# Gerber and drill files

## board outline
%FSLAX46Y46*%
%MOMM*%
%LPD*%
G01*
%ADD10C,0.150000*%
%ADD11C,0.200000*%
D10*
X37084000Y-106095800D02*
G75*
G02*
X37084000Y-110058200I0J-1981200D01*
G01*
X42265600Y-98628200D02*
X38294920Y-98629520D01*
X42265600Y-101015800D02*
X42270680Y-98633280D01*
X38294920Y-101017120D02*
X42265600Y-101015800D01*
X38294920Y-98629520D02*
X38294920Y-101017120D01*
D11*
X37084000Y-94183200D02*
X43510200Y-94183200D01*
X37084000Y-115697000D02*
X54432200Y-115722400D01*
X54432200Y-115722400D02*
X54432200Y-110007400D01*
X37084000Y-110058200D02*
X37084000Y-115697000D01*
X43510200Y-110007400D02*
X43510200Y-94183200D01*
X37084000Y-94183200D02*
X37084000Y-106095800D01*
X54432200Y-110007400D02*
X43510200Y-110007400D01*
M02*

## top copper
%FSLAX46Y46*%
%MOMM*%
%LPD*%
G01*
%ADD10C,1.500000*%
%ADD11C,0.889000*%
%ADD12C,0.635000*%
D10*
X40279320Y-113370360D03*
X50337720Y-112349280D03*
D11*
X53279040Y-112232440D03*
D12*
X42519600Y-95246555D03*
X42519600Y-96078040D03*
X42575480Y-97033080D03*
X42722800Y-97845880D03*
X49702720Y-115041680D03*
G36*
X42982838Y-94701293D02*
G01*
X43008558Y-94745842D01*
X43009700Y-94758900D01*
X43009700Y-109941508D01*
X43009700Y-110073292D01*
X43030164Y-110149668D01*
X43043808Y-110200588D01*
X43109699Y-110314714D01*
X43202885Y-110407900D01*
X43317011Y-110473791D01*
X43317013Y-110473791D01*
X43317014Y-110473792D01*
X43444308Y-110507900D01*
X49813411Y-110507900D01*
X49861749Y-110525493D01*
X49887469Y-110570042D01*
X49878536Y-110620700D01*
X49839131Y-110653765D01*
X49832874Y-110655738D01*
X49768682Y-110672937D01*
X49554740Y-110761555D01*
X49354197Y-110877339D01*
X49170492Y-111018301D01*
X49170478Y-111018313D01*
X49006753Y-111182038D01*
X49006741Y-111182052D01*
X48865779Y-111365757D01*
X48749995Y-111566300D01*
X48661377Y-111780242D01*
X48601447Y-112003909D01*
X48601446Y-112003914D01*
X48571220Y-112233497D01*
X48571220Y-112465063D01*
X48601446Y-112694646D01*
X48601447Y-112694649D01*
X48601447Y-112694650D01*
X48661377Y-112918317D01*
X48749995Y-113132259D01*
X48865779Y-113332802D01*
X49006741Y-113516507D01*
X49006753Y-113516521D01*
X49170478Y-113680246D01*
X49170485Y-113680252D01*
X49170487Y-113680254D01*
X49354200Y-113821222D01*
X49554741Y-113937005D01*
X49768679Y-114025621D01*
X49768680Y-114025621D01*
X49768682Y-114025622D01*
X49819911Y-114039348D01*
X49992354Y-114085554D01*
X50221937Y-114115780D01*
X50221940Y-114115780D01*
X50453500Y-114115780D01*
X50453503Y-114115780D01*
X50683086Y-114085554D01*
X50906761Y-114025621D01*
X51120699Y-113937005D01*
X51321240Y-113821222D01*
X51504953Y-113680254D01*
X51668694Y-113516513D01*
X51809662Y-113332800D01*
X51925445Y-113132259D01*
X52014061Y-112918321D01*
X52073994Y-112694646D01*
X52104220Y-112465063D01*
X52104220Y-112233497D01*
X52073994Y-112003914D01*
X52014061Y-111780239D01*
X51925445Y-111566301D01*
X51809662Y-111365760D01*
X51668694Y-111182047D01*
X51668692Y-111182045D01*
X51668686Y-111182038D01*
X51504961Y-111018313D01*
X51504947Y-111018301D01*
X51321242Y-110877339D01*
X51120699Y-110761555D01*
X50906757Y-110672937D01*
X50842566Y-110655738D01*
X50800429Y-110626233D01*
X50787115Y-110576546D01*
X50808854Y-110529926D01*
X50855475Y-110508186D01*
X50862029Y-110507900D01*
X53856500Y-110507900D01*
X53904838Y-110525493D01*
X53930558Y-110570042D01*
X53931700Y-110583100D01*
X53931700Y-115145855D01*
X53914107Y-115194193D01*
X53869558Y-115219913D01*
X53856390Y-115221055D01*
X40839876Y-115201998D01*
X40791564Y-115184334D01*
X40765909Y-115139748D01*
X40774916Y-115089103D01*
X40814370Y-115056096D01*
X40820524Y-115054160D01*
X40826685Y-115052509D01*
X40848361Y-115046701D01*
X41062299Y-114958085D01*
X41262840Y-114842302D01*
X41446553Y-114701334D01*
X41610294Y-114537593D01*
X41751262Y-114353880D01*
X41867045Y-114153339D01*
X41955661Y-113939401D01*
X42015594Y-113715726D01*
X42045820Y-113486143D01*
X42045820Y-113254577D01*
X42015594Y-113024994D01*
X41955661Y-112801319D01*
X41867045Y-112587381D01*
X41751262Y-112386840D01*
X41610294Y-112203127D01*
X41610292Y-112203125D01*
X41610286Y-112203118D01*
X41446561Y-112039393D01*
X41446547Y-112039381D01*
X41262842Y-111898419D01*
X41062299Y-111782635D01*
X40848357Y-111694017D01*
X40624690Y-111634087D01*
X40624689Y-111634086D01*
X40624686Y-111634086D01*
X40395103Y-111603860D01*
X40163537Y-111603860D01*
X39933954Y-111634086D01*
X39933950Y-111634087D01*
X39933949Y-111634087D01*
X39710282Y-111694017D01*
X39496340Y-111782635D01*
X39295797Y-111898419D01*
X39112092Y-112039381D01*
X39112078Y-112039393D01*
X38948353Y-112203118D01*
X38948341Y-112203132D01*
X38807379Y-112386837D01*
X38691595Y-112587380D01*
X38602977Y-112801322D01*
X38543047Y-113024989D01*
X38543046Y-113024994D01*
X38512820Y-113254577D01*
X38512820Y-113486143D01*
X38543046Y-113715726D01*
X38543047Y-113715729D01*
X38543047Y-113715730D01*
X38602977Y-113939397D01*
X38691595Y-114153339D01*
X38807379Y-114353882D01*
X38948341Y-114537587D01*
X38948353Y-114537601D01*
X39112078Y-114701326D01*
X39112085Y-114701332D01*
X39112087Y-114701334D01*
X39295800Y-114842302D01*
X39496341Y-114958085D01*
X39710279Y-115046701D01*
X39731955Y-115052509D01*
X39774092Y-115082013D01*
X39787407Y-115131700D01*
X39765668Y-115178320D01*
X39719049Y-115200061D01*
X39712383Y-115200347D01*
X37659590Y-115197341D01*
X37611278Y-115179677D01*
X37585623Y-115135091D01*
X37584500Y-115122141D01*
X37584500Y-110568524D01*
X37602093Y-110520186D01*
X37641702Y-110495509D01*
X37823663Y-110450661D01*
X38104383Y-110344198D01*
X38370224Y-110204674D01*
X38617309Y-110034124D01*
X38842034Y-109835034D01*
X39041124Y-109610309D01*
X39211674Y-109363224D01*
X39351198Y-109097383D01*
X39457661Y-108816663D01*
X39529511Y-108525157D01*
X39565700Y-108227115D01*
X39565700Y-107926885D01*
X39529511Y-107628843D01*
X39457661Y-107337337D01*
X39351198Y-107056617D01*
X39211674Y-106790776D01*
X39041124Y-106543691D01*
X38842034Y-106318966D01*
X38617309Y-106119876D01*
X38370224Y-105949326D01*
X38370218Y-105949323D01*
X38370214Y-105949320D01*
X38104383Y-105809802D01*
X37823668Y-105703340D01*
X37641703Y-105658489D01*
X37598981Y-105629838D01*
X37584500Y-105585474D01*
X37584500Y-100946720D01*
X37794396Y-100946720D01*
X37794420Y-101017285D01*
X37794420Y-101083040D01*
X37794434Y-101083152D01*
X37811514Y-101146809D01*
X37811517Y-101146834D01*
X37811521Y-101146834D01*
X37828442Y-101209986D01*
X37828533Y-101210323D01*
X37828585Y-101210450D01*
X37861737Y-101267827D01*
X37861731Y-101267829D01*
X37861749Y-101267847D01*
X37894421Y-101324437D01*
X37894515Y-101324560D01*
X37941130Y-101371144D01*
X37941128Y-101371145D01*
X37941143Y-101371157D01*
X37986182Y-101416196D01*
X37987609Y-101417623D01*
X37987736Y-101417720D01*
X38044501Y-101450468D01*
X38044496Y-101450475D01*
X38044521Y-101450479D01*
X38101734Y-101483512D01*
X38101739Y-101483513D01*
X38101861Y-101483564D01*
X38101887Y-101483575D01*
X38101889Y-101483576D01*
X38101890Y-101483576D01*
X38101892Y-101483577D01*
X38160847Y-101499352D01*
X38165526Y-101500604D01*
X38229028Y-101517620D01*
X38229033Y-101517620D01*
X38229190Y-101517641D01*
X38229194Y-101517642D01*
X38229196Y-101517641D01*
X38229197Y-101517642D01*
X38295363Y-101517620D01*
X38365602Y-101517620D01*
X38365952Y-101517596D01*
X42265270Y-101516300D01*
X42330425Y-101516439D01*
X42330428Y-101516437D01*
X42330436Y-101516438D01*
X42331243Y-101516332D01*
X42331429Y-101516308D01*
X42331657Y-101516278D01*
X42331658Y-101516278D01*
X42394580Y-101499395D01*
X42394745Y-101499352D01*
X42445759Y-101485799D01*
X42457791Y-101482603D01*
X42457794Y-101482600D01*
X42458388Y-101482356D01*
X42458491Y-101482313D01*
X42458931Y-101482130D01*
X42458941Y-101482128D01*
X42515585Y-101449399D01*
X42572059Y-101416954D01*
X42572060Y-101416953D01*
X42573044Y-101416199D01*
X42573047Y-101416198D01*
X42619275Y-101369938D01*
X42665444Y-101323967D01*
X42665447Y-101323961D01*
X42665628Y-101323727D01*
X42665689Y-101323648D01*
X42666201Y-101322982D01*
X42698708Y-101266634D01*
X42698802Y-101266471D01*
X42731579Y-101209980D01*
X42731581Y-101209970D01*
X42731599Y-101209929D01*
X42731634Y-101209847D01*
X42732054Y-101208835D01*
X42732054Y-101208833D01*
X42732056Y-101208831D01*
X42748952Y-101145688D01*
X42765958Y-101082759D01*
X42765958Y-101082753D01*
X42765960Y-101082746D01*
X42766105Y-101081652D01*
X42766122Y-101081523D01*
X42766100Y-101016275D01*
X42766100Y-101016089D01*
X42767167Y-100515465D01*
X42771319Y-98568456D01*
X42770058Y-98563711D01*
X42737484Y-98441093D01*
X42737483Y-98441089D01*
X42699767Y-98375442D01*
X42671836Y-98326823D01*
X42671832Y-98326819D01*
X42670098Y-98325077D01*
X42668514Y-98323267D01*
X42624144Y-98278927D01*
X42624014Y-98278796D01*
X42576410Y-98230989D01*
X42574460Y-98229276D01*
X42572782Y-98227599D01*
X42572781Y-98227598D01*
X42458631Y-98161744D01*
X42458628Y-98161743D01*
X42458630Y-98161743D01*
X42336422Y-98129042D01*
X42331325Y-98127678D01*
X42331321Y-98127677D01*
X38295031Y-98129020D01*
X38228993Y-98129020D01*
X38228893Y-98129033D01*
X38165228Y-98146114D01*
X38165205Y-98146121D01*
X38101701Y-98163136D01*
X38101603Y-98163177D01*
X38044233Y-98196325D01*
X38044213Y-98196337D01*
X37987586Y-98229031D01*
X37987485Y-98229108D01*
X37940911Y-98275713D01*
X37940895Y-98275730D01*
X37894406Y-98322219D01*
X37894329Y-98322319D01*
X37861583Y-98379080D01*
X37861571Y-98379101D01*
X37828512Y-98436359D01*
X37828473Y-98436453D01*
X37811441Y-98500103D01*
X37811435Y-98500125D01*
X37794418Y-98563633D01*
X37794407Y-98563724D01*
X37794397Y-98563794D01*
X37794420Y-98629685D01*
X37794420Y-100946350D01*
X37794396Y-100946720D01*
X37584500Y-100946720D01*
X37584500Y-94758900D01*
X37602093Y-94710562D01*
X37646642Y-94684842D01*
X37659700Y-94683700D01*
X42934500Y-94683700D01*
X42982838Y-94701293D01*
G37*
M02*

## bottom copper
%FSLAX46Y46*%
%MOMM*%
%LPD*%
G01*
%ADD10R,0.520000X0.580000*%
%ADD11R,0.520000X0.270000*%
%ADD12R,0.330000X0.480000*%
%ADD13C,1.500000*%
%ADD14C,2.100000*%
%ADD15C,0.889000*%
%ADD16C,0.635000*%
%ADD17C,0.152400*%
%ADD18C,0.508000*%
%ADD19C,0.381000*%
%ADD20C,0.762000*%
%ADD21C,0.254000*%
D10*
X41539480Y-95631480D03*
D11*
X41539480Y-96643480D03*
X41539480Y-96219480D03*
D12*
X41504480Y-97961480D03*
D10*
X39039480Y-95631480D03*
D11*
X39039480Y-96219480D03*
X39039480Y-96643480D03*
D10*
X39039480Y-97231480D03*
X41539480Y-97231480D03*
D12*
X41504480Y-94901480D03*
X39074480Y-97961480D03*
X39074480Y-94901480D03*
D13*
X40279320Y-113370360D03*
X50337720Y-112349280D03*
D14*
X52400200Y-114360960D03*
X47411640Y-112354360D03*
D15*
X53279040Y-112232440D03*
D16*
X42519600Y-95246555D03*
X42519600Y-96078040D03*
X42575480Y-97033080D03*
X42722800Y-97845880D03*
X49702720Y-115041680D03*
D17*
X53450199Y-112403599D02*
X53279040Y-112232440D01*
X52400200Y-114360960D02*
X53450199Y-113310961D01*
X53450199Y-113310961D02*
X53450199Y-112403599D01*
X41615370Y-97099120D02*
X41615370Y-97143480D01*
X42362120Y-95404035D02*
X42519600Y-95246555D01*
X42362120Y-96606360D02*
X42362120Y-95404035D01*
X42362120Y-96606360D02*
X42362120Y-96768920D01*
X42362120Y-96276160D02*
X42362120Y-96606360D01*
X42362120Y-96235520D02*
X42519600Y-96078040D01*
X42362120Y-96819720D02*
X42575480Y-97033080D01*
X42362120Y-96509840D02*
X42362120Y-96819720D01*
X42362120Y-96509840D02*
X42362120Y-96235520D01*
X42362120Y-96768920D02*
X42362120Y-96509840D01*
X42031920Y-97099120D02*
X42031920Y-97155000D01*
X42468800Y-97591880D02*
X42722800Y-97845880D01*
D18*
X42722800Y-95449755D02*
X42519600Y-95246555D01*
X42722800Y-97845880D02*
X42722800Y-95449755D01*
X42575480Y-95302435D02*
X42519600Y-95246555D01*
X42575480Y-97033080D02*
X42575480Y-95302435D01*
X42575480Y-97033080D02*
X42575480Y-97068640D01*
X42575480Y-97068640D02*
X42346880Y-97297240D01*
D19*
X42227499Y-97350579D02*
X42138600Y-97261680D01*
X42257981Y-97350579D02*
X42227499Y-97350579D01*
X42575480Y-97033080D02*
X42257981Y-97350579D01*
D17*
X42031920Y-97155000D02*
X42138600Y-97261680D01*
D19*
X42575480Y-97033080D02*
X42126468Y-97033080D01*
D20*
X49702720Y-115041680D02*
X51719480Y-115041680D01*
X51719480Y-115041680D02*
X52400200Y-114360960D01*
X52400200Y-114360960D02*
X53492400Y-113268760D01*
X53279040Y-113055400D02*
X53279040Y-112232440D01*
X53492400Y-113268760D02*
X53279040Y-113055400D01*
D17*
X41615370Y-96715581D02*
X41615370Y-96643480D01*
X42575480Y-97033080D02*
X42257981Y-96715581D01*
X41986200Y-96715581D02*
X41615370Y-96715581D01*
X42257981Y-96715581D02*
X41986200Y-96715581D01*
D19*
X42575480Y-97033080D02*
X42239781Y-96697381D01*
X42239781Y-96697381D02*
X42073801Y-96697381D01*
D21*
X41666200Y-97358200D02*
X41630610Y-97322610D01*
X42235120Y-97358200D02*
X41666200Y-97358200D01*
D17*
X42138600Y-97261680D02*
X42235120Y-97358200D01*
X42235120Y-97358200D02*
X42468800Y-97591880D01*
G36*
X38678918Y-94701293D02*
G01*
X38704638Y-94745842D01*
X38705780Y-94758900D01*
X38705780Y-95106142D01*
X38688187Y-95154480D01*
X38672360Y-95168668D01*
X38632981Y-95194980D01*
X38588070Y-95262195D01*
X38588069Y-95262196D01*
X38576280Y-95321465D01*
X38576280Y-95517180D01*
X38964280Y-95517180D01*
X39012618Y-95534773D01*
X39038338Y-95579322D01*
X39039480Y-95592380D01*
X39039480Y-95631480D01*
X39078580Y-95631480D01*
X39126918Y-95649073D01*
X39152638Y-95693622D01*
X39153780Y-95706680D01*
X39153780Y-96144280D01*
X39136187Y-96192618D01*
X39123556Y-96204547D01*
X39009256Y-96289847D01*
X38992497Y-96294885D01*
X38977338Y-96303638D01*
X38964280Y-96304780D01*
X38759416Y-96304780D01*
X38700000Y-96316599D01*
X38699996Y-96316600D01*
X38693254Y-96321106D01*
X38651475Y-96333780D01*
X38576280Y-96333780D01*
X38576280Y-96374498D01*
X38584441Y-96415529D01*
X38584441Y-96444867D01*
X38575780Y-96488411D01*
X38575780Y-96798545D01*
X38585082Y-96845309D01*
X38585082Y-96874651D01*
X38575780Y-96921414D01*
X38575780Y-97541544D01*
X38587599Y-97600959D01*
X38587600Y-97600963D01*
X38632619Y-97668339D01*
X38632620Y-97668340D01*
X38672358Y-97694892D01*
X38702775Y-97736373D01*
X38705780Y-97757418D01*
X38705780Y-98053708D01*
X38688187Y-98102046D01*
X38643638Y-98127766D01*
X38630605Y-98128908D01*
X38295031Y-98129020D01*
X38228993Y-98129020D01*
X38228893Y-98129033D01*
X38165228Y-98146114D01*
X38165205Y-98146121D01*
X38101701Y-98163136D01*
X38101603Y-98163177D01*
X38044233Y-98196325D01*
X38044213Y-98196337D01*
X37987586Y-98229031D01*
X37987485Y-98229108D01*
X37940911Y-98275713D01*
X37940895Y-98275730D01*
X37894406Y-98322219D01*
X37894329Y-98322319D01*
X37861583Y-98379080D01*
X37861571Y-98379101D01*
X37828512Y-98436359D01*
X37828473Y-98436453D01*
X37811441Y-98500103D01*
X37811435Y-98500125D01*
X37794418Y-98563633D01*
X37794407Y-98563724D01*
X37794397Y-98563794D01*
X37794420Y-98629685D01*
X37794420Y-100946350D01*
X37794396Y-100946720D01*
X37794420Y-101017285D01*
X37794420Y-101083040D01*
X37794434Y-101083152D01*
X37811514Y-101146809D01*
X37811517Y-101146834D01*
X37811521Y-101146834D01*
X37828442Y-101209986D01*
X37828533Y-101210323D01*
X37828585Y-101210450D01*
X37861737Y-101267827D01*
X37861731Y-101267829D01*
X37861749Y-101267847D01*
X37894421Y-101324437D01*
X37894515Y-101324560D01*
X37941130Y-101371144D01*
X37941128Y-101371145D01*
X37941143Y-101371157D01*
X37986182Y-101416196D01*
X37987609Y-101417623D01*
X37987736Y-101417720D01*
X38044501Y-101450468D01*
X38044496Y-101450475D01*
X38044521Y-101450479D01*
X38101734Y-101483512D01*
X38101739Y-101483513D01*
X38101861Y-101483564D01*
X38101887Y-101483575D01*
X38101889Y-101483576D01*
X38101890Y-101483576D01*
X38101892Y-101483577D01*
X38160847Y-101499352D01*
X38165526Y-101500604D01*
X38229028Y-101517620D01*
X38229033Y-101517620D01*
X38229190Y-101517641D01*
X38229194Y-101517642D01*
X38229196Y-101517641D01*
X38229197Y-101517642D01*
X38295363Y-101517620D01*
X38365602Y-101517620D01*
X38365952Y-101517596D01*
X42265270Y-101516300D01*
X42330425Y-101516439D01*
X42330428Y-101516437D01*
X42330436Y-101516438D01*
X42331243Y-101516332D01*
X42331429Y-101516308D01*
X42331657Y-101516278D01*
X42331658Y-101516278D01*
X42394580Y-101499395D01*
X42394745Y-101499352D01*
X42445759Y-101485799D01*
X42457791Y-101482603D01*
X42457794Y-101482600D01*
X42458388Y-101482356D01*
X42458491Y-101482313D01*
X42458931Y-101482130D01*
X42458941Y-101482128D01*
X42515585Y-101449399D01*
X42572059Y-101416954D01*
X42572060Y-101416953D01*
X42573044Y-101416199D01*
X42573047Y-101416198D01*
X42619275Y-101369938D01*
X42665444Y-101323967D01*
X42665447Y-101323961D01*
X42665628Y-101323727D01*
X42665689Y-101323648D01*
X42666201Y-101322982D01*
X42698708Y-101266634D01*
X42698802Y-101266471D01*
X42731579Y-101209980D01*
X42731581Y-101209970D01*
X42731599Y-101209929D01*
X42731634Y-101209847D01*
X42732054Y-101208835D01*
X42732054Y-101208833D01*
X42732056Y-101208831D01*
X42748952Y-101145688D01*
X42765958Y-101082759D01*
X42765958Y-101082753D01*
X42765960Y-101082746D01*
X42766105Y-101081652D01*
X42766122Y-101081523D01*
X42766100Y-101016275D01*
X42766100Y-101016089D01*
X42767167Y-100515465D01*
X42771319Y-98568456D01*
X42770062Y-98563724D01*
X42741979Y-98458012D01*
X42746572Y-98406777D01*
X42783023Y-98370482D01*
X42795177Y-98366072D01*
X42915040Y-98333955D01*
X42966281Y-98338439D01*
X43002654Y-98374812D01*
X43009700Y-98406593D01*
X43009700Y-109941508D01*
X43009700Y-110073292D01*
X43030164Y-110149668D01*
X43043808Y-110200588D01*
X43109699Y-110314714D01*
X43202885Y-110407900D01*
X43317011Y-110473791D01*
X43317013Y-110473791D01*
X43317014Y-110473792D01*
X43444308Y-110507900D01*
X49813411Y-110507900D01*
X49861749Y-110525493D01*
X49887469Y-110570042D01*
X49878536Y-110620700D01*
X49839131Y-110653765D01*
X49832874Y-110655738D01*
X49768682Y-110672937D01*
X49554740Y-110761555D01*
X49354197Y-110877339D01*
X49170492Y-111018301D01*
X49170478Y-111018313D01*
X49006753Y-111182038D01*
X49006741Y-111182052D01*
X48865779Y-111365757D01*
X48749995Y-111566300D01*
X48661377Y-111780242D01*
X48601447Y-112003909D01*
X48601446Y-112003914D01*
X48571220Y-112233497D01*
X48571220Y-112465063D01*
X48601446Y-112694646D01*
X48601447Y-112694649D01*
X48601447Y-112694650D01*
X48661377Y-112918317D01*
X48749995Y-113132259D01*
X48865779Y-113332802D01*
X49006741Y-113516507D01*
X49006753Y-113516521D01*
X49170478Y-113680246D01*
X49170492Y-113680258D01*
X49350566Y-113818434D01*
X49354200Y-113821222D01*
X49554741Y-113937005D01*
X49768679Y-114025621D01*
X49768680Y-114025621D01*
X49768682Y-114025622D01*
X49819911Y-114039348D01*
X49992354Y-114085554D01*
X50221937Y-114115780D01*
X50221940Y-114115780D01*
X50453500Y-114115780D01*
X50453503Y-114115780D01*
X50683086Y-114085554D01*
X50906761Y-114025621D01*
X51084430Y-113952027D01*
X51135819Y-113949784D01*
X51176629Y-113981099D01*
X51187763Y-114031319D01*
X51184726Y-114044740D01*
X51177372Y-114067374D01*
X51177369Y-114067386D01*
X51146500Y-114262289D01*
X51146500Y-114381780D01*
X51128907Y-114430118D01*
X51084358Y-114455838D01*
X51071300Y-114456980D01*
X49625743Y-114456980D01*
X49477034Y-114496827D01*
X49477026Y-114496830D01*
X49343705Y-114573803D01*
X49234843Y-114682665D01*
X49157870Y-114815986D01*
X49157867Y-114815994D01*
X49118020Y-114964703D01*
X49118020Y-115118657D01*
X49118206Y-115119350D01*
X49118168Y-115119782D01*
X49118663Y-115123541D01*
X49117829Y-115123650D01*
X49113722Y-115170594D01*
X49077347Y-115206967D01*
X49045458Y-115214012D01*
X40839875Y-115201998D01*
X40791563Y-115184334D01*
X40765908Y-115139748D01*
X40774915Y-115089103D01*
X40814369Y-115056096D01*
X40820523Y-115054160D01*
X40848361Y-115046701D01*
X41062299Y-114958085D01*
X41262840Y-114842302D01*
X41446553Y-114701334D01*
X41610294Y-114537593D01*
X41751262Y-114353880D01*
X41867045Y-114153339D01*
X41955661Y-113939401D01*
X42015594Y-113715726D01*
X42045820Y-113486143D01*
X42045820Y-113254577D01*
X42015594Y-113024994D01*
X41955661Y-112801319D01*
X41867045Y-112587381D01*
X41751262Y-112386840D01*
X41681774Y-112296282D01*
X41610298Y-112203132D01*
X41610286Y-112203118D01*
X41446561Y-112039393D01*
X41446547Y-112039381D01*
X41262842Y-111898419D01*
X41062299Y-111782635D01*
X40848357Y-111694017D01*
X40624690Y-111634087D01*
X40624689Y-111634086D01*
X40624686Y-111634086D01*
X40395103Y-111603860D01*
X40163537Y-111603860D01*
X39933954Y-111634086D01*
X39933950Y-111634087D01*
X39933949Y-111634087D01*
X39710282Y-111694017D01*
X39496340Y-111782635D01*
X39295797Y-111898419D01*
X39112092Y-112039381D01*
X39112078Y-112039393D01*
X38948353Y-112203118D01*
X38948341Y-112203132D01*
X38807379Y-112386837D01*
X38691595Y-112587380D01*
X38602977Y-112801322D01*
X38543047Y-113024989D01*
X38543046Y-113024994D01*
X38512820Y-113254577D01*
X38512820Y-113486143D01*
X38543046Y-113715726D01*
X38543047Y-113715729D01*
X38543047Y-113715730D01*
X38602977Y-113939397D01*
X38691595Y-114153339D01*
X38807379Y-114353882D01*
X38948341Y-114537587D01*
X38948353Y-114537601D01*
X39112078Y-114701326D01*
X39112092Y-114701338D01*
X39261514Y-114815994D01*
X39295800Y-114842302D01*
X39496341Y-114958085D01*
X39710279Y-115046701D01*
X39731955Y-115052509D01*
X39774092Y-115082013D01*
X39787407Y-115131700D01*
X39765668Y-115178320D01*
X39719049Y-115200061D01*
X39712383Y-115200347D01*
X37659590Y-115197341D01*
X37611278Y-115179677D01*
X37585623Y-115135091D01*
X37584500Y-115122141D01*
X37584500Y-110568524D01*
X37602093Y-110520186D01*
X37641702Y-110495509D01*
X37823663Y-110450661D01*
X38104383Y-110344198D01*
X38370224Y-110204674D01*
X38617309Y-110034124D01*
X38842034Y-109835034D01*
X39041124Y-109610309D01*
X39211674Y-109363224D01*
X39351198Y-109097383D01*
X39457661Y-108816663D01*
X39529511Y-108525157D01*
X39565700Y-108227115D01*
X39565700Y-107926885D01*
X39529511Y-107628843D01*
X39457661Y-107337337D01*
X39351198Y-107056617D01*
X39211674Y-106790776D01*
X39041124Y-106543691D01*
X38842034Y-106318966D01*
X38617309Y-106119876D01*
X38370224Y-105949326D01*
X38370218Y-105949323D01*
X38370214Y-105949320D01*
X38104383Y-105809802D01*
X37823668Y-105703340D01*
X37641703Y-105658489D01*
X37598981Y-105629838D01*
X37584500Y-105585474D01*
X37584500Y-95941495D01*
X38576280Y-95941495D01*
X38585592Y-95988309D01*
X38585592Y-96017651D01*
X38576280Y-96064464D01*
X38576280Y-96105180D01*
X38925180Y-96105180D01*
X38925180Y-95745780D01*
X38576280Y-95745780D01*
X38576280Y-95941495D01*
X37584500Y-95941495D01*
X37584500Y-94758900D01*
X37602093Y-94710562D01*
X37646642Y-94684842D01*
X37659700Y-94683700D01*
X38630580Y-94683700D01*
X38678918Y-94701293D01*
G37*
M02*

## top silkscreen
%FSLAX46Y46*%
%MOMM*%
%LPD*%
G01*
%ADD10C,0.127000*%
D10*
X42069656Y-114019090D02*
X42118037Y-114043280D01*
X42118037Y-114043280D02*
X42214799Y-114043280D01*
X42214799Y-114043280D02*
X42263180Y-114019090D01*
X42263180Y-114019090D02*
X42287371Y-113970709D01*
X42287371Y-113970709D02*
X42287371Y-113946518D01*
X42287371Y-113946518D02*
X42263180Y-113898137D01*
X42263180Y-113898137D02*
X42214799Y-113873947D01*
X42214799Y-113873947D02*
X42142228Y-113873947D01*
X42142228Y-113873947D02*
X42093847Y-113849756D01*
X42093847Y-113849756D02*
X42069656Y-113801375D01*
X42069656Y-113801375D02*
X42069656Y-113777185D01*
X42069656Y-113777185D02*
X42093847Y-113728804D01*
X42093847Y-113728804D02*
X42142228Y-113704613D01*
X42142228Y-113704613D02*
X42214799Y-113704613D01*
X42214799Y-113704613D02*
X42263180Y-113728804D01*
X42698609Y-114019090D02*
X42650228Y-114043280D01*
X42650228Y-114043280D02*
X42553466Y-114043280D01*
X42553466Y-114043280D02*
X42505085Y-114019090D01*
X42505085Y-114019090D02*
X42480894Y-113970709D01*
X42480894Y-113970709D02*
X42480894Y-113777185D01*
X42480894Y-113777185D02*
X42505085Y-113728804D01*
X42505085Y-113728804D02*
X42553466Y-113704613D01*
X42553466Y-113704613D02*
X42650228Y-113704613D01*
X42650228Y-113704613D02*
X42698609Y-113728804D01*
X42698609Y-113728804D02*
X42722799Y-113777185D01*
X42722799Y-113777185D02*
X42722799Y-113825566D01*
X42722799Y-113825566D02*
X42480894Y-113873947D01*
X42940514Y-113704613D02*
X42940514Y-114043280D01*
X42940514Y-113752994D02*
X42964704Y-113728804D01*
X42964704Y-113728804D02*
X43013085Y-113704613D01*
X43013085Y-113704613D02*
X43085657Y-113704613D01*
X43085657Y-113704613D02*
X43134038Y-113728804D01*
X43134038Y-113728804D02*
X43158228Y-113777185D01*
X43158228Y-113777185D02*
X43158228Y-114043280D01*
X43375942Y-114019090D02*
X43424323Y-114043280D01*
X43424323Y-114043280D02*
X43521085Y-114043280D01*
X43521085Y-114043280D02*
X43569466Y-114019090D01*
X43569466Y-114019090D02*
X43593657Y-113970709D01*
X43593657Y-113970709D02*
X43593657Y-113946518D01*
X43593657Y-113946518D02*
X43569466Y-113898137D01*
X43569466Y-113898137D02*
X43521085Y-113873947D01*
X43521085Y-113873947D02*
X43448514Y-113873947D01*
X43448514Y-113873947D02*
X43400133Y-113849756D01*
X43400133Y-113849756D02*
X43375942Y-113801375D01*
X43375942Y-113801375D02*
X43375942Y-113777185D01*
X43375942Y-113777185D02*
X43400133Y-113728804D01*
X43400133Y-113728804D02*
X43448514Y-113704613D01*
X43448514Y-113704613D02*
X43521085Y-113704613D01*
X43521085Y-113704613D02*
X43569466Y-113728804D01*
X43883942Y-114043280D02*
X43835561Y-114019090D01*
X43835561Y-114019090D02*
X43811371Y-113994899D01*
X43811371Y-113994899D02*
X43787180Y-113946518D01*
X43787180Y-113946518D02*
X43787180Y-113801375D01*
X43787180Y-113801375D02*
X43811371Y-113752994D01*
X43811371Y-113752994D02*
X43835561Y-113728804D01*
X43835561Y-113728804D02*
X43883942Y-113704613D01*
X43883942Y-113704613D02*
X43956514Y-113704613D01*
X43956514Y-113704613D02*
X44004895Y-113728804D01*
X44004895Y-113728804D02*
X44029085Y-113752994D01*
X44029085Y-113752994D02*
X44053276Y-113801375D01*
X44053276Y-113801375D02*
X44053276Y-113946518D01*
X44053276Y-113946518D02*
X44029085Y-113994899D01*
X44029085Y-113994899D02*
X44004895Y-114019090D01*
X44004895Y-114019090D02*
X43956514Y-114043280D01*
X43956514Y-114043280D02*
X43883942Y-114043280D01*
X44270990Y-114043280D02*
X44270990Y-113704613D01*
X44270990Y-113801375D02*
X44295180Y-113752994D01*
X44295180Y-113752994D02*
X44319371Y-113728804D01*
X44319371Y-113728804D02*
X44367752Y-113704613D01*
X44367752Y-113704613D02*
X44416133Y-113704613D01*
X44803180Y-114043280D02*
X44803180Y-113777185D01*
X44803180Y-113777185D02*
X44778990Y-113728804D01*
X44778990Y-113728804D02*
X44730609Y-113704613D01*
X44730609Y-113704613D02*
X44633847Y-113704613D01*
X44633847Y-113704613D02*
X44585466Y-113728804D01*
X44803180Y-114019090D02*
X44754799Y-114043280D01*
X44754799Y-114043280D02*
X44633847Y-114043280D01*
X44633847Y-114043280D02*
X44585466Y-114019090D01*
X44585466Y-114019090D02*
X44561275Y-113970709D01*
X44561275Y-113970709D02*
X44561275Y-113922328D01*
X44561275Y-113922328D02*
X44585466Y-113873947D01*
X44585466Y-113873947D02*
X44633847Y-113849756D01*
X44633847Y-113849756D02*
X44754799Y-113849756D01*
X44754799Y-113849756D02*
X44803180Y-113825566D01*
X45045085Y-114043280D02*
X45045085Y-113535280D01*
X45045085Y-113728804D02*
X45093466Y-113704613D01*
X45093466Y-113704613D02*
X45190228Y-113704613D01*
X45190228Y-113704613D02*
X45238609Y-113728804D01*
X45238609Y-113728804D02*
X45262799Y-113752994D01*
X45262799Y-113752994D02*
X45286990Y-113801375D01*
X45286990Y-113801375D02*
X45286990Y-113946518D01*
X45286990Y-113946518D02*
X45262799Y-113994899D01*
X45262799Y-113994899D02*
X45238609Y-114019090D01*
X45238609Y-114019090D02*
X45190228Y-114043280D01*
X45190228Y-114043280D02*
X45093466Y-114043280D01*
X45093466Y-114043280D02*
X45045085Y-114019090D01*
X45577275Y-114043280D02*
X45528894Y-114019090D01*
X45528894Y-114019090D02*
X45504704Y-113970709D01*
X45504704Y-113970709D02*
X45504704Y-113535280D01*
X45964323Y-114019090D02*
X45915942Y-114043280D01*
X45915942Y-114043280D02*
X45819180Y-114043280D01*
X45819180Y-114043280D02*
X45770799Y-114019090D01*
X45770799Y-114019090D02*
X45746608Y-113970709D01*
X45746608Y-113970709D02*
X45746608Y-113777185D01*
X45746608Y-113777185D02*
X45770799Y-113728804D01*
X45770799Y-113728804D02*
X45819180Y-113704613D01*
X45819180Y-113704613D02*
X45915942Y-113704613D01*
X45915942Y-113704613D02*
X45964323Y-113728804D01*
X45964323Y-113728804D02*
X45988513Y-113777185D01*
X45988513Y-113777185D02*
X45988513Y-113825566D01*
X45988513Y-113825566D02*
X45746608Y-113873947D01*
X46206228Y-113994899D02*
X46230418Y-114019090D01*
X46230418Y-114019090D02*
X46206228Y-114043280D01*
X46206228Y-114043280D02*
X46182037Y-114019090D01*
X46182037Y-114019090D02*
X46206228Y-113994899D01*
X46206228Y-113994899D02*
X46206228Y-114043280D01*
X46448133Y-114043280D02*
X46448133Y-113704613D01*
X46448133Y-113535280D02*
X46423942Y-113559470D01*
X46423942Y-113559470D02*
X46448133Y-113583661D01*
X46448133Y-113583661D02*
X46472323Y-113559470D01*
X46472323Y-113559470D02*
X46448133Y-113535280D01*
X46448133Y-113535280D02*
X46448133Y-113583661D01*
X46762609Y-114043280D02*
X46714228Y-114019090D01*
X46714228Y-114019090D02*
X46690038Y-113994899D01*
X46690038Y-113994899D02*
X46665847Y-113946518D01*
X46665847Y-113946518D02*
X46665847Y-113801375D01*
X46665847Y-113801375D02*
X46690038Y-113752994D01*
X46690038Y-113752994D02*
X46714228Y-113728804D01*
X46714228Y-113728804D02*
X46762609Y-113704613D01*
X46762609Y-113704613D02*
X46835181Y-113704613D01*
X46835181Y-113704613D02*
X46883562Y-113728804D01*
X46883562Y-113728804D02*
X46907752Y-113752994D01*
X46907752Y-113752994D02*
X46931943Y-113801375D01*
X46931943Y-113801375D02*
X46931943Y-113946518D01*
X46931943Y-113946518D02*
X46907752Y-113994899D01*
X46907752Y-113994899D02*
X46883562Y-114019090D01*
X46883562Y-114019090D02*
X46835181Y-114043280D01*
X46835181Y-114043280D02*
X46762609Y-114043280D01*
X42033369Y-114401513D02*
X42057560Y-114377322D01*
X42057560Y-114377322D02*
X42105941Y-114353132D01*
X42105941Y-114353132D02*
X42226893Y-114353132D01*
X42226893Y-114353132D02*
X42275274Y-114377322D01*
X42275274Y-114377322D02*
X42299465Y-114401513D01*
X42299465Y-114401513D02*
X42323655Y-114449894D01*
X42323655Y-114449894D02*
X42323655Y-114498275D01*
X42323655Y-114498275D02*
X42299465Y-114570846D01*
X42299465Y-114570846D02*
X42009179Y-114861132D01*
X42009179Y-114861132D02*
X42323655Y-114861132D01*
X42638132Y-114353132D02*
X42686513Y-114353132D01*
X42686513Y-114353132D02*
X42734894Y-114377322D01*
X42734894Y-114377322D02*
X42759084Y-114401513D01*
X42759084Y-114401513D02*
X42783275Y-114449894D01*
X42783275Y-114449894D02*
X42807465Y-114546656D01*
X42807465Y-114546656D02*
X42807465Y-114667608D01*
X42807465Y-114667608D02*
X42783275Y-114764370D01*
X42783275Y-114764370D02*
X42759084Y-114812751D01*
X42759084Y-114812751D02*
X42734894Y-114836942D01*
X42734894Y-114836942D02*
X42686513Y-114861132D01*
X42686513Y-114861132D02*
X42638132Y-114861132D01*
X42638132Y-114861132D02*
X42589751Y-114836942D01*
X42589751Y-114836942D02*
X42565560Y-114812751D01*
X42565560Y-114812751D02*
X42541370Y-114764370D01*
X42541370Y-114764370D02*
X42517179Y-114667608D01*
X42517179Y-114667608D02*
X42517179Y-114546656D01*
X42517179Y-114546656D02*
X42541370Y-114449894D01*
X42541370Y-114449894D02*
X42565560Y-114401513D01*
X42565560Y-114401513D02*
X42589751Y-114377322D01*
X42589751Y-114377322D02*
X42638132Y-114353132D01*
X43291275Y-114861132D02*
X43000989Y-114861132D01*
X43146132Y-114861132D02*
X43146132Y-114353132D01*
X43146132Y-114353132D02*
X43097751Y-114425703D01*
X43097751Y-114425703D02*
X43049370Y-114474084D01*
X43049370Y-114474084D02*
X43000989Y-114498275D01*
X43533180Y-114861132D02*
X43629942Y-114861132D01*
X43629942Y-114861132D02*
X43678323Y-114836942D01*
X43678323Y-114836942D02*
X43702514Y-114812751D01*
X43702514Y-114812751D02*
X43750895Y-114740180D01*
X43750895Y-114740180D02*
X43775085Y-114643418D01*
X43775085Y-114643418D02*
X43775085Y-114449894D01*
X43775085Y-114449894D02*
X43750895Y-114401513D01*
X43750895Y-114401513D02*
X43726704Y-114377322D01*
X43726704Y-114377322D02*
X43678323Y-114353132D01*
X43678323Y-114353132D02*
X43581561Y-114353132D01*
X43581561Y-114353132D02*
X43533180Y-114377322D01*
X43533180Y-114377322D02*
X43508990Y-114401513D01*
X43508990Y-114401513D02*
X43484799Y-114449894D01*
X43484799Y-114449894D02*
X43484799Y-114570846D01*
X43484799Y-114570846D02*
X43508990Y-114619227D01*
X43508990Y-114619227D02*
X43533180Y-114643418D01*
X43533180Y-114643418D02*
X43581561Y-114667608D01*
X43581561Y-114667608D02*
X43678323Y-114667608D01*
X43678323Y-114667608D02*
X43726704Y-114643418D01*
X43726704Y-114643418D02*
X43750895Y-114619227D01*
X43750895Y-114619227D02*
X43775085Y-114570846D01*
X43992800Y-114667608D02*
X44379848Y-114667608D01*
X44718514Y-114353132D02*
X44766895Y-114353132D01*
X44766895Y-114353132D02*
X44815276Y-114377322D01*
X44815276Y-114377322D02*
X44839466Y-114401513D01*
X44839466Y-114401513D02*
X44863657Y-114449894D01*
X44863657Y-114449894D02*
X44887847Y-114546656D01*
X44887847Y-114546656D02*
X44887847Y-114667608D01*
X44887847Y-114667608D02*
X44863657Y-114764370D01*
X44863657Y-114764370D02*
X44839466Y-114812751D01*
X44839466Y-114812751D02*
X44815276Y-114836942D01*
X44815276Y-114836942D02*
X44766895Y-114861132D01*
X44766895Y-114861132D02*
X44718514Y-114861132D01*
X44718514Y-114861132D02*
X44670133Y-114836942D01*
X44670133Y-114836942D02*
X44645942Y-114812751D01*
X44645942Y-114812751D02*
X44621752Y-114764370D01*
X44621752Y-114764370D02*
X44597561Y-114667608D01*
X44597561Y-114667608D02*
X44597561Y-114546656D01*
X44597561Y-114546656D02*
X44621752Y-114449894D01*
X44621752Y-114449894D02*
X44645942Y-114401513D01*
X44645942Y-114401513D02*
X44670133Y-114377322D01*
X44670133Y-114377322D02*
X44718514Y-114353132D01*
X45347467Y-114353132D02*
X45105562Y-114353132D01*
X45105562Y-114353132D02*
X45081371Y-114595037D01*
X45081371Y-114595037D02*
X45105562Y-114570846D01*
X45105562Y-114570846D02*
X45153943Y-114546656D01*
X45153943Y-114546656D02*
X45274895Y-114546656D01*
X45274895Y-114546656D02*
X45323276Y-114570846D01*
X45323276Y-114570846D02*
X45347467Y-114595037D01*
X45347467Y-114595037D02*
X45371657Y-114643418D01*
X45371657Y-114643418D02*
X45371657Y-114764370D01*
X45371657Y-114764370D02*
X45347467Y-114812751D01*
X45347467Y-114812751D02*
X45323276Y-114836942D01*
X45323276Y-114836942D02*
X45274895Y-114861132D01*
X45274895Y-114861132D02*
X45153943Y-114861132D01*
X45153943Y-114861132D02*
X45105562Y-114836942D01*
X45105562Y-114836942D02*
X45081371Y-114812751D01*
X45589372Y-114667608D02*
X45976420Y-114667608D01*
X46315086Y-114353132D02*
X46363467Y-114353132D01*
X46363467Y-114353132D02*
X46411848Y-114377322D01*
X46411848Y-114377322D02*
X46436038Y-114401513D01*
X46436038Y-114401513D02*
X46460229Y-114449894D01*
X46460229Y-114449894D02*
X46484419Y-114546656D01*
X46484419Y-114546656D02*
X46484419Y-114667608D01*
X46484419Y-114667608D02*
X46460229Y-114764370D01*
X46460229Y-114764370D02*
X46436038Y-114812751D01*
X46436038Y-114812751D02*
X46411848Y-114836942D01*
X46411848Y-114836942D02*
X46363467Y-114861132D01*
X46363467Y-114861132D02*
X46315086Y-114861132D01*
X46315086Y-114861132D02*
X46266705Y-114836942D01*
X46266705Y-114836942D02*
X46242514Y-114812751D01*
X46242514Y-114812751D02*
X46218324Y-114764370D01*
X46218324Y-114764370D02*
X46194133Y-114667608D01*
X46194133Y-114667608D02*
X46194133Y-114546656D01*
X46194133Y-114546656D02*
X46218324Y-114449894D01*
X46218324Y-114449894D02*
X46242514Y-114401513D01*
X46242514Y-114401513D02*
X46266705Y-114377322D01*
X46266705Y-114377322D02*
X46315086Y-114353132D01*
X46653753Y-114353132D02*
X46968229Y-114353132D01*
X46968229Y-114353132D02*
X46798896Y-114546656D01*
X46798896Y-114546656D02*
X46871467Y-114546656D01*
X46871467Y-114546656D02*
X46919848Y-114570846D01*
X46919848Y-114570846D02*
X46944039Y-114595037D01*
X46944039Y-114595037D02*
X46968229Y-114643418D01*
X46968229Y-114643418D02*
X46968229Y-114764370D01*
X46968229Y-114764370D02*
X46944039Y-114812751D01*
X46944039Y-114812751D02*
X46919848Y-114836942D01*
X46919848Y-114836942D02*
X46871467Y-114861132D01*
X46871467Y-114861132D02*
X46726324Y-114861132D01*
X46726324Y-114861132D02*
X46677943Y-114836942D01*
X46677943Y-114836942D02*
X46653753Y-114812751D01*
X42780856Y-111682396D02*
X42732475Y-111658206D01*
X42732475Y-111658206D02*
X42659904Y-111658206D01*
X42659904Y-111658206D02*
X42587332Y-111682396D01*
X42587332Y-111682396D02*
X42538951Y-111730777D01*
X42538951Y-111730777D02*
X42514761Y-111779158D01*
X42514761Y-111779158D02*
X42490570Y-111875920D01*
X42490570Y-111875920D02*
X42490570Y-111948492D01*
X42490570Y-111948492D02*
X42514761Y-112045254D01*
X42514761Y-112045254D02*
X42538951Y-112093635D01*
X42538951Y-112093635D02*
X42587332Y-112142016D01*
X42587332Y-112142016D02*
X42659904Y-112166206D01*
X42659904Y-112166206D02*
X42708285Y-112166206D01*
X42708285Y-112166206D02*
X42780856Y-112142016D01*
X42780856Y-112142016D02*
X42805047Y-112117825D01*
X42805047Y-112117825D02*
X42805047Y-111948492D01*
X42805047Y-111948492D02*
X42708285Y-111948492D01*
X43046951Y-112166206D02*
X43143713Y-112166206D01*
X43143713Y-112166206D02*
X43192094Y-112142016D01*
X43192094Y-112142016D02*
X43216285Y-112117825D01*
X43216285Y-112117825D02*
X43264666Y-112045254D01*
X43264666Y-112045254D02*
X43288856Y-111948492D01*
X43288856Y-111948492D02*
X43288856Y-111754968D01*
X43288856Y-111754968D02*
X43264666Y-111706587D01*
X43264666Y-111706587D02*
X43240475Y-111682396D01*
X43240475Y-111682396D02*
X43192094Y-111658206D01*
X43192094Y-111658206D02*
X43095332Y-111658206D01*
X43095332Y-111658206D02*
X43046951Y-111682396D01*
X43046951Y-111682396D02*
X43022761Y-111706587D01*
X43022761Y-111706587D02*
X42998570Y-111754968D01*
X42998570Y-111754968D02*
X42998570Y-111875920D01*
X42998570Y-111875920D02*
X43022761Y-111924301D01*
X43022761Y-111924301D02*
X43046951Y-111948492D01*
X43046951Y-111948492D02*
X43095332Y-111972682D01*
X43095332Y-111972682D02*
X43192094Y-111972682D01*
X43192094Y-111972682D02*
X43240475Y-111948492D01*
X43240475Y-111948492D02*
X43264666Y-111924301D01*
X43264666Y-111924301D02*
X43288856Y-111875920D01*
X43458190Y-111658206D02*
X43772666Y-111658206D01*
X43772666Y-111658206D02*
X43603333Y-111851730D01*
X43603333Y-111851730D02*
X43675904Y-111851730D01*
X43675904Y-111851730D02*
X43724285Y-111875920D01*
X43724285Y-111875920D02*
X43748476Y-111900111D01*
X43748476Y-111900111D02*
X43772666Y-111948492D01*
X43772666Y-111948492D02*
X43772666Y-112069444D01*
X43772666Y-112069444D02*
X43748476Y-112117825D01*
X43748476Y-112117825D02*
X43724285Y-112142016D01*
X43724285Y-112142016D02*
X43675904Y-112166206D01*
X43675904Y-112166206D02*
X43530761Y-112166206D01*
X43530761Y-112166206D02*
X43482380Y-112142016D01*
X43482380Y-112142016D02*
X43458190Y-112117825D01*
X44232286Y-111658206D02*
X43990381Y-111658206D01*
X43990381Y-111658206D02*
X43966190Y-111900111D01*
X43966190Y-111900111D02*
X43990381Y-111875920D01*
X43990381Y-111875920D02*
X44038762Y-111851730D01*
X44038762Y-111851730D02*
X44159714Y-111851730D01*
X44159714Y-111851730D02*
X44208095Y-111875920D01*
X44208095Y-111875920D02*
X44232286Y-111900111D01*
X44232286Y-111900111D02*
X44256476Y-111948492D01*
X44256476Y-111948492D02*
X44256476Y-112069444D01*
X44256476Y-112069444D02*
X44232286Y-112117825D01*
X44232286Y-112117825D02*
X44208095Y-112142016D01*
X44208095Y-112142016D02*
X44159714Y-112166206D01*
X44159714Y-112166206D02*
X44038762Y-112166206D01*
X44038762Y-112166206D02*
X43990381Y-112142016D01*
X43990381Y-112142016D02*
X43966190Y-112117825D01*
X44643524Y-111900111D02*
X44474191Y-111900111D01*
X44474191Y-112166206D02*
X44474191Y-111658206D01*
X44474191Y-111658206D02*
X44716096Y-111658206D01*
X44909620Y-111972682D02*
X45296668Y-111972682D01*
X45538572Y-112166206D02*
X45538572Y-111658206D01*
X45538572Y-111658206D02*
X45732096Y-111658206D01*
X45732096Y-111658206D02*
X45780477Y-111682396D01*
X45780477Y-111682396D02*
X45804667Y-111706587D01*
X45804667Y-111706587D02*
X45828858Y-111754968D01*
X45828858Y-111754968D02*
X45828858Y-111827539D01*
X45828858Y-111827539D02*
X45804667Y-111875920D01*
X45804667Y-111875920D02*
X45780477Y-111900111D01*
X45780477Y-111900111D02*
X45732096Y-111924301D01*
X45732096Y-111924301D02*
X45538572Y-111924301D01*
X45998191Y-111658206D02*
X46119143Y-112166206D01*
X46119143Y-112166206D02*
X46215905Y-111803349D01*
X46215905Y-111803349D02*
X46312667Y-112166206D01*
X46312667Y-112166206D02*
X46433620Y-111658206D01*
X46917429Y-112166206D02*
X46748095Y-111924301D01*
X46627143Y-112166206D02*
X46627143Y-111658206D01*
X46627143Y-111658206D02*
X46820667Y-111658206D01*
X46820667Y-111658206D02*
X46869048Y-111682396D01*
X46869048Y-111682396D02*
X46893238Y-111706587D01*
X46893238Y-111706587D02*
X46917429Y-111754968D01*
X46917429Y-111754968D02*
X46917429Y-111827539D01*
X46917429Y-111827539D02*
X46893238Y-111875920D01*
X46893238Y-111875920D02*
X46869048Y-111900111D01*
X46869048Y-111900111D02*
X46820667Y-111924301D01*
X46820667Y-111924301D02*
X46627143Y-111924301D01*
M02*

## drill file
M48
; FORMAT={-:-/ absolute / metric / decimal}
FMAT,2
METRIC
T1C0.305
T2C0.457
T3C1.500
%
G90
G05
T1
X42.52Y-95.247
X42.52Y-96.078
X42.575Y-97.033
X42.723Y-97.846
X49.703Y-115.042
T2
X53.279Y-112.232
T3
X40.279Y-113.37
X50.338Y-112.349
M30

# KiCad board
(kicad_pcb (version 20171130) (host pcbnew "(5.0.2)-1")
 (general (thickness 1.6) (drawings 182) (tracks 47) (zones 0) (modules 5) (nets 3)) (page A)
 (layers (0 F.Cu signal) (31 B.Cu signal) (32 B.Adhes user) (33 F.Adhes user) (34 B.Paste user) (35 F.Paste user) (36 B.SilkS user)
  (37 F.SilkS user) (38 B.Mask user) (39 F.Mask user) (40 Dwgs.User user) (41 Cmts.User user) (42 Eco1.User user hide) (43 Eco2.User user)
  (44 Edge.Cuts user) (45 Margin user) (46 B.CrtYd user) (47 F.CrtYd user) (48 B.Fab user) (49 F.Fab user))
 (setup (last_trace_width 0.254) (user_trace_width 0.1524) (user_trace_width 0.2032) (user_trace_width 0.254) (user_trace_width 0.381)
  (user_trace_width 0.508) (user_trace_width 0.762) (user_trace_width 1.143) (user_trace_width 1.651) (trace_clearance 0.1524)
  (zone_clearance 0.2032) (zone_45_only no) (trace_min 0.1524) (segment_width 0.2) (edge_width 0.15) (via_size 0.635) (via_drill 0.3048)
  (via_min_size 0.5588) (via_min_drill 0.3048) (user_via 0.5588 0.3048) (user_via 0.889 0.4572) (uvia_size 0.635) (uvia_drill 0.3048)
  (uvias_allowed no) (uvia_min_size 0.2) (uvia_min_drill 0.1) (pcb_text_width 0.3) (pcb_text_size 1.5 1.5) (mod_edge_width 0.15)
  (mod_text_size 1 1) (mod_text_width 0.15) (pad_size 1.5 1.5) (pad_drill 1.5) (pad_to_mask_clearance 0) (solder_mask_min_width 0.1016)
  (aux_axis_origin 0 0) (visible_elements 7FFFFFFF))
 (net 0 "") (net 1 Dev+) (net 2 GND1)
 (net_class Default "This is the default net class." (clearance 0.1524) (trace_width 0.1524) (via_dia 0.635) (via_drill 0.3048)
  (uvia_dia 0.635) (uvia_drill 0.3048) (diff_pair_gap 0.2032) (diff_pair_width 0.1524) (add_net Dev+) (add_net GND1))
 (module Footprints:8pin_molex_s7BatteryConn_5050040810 (layer B.Cu) (at 40.28948 96.43148)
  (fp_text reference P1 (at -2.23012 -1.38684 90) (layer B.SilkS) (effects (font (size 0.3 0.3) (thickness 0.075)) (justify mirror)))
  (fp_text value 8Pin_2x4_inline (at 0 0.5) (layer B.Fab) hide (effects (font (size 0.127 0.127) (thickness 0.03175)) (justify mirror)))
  (pad 5 smd rect (at 1.25 -0.8) (size 0.52 0.58) (layers B.Cu B.Paste B.Mask))
  (pad 7 smd rect (at 1.25 0.212) (size 0.52 0.27) (layers B.Cu B.Paste B.Mask) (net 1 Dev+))
  (pad 6 smd rect (at 1.25 -0.212) (size 0.52 0.27) (layers B.Cu B.Paste B.Mask))
  (pad "" smd rect (at 1.215 1.53) (size 0.33 0.48) (layers B.Cu B.Paste B.Mask))
  (pad 4 smd rect (at -1.25 -0.8) (size 0.52 0.58) (layers B.Cu B.Paste B.Mask) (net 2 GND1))
  (pad 3 smd rect (at -1.25 -0.212) (size 0.52 0.27) (layers B.Cu B.Paste B.Mask) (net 2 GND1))
  (pad 2 smd rect (at -1.25 0.212) (size 0.52 0.27) (layers B.Cu B.Paste B.Mask))
  (pad 1 smd rect (at -1.25 0.8) (size 0.52 0.58) (layers B.Cu B.Paste B.Mask))
  (pad 8 smd rect (at 1.25 0.8) (size 0.52 0.58) (layers B.Cu B.Paste B.Mask) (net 1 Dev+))
  (pad "" smd rect (at 1.215 -1.53) (size 0.33 0.48) (layers B.Cu B.Paste B.Mask))
  (pad "" smd rect (at -1.215 1.53) (size 0.33 0.48) (layers B.Cu B.Paste B.Mask))
  (pad "" smd rect (at -1.215 -1.53) (size 0.33 0.48) (layers B.Cu B.Paste B.Mask)))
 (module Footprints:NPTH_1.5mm (layer F.Cu) (at 40.27932 113.37036)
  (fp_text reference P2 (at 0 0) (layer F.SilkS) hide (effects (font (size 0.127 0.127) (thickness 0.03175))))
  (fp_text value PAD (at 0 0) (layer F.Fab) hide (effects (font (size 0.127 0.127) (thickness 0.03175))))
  (pad "" thru_hole circle (at 0 0) (size 1.5 1.5) (drill 1.5) (layers *.Cu *.Mask) (clearance 1.016)))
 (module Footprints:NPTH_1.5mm (layer F.Cu) (at 50.33772 112.34928)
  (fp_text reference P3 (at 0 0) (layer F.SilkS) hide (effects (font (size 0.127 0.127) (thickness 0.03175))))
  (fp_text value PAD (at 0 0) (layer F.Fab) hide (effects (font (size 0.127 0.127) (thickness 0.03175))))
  (pad "" thru_hole circle (at 0 0) (size 1.5 1.5) (drill 1.5) (layers *.Cu *.Mask) (clearance 1.016)))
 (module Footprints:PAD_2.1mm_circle (layer B.Cu) (at 52.4002 114.36096)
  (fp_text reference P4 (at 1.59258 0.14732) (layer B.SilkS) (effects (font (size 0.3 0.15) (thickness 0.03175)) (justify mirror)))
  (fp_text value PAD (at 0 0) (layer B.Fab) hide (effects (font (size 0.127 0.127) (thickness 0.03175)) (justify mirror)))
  (pad 1 smd circle (at 0 0) (size 2.1 2.1) (layers B.Cu B.Paste B.Mask) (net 1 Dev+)))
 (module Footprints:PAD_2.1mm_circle (layer B.Cu) (at 47.41164 112.35436)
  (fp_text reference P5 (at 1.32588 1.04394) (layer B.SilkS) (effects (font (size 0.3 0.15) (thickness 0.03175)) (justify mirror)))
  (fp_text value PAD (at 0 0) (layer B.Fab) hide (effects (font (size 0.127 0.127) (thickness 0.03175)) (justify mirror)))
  (pad 1 smd circle (at 0 0) (size 2.1 2.1) (layers B.Cu B.Paste B.Mask) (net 2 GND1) (zone_connect 2)))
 (gr_arc (start 37.084 108.077) (end 37.084 110.0582) (angle -180) (layer Edge.Cuts) (width 0.15))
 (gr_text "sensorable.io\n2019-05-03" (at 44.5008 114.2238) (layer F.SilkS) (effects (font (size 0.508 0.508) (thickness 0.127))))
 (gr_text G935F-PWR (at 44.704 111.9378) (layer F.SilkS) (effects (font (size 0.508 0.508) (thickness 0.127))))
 (gr_line (start 42.2656 98.6282) (end 38.29492 98.62952) (layer Edge.Cuts) (width 0.15))
 (gr_line (start 42.2656 101.0158) (end 42.27068 98.63328) (layer Edge.Cuts) (width 0.15))
 (gr_line (start 38.29492 101.01712) (end 42.2656 101.0158) (layer Edge.Cuts) (width 0.15))
 (gr_line (start 38.29492 98.62952) (end 38.29492 101.01712) (layer Edge.Cuts) (width 0.15))
 (gr_line (start 37.084 94.1832) (end 43.5102 94.1832) (layer Edge.Cuts) (width 0.2))
 (gr_line (start 37.084 115.697) (end 54.4322 115.7224) (layer Edge.Cuts) (width 0.2))
 (gr_line (start 54.4322 115.7224) (end 54.4322 110.0074) (layer Edge.Cuts) (width 0.2))
 (gr_line (start 37.084 110.0582) (end 37.084 115.697) (layer Edge.Cuts) (width 0.2))
 (gr_line (start 43.5102 110.0074) (end 43.5102 94.1832) (layer Edge.Cuts) (width 0.2))
 (gr_line (start 37.084 94.1832) (end 37.084 106.0958) (layer Edge.Cuts) (width 0.2))
 (gr_line (start 54.4322 110.0074) (end 43.5102 110.0074) (layer Edge.Cuts) (width 0.2))
 (via (at 53.27904 112.23244) (size 0.889) (drill 0.4572) (layers F.Cu B.Cu) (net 1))
 (segment (start 53.450199 112.403599) (end 53.27904 112.23244) (width 0.1524) (layer B.Cu) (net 1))
 (segment (start 52.4002 114.36096) (end 53.450199 113.310961) (width 0.1524) (layer B.Cu) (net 1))
 (segment (start 53.450199 113.310961) (end 53.450199 112.403599) (width 0.1524) (layer B.Cu) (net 1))
 (segment (start 41.61537 97.09912) (end 41.61537 97.14348) (width 0.1524) (layer B.Cu) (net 1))
 (via (at 42.5196 95.246555) (size 0.635) (drill 0.3048) (layers F.Cu B.Cu) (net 1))
 (segment (start 42.36212 95.404035) (end 42.5196 95.246555) (width 0.1524) (layer B.Cu) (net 1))
 (segment (start 42.36212 96.60636) (end 42.36212 95.404035) (width 0.1524) (layer B.Cu) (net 1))
 (segment (start 42.36212 96.60636) (end 42.36212 96.76892) (width 0.1524) (layer B.Cu) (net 1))
 (segment (start 42.36212 96.27616) (end 42.36212 96.60636) (width 0.1524) (layer B.Cu) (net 1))
 (via (at 42.5196 96.07804) (size 0.635) (drill 0.3048) (layers F.Cu B.Cu) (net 1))
 (segment (start 42.36212 96.23552) (end 42.5196 96.07804) (width 0.1524) (layer B.Cu) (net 1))
 (via (at 42.57548 97.03308) (size 0.635) (drill 0.3048) (layers F.Cu B.Cu) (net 1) (status 1000000))
 (segment (start 42.36212 96.81972) (end 42.57548 97.03308) (width 0.1524) (layer B.Cu) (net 1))
 (segment (start 42.36212 96.50984) (end 42.36212 96.81972) (width 0.1524) (layer B.Cu) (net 1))
 (segment (start 42.36212 96.50984) (end 42.36212 96.23552) (width 0.1524) (layer B.Cu) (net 1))
 (segment (start 42.36212 96.76892) (end 42.36212 96.50984) (width 0.1524) (layer B.Cu) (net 1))
 (segment (start 42.03192 97.09912) (end 42.03192 97.155) (width 0.1524) (layer B.Cu) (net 1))
 (segment (start 42.4688 97.59188) (end 42.7228 97.84588) (width 0.1524) (layer B.Cu) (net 1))
 (via (at 42.7228 97.84588) (size 0.635) (drill 0.3048) (layers F.Cu B.Cu) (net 1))
 (segment (start 42.7228 95.449755) (end 42.5196 95.246555) (width 0.508) (layer B.Cu) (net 1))
 (segment (start 42.7228 97.84588) (end 42.7228 95.449755) (width 0.508) (layer B.Cu) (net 1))
 (segment (start 42.57548 95.302435) (end 42.5196 95.246555) (width 0.508) (layer B.Cu) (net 1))
 (segment (start 42.57548 97.03308) (end 42.57548 95.302435) (width 0.508) (layer B.Cu) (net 1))
 (segment (start 42.57548 97.03308) (end 42.57548 97.06864) (width 0.508) (layer B.Cu) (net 1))
 (segment (start 42.57548 97.06864) (end 42.34688 97.29724) (width 0.508) (layer B.Cu) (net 1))
 (segment (start 42.227499 97.350579) (end 42.1386 97.26168) (width 0.381) (layer B.Cu) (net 1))
 (segment (start 42.257981 97.350579) (end 42.227499 97.350579) (width 0.381) (layer B.Cu) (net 1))
 (segment (start 42.57548 97.03308) (end 42.257981 97.350579) (width 0.381) (layer B.Cu) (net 1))
 (segment (start 42.03192 97.155) (end 42.1386 97.26168) (width 0.1524) (layer B.Cu) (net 1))
 (segment (start 42.57548 97.03308) (end 42.126468 97.03308) (width 0.381) (layer B.Cu) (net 1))
 (via (at 49.70272 115.04168) (size 0.635) (drill 0.3048) (layers F.Cu B.Cu) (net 1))
 (segment (start 49.70272 115.04168) (end 51.71948 115.04168) (width 0.762) (layer B.Cu) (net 1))
 (segment (start 51.71948 115.04168) (end 52.4002 114.36096) (width 0.762) (layer B.Cu) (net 1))
 (segment (start 52.4002 114.36096) (end 53.4924 113.26876) (width 0.762) (layer B.Cu) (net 1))
 (segment (start 53.27904 113.0554) (end 53.27904 112.23244) (width 0.762) (layer B.Cu) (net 1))
 (segment (start 53.4924 113.26876) (end 53.27904 113.0554) (width 0.762) (layer B.Cu) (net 1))
 (segment (start 41.61537 96.715581) (end 41.61537 96.64348) (width 0.1524) (layer B.Cu) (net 1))
 (segment (start 42.57548 97.03308) (end 42.257981 96.715581) (width 0.1524) (layer B.Cu) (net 1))
 (segment (start 41.9862 96.715581) (end 41.61537 96.715581) (width 0.1524) (layer B.Cu) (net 1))
 (segment (start 42.257981 96.715581) (end 41.9862 96.715581) (width 0.1524) (layer B.Cu) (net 1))
 (segment (start 42.57548 97.03308) (end 42.239781 96.697381) (width 0.381) (layer B.Cu) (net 1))
 (segment (start 42.239781 96.697381) (end 42.073801 96.697381) (width 0.381) (layer B.Cu) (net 1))
 (segment (start 41.6662 97.3582) (end 41.63061 97.32261) (width 0.254) (layer B.Cu) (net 1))
 (segment (start 42.23512 97.3582) (end 41.6662 97.3582) (width 0.254) (layer B.Cu) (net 1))
 (segment (start 42.1386 97.26168) (end 42.23512 97.3582) (width 0.1524) (layer B.Cu) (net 1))
 (segment (start 42.23512 97.3582) (end 42.4688 97.59188) (width 0.1524) (layer B.Cu) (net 1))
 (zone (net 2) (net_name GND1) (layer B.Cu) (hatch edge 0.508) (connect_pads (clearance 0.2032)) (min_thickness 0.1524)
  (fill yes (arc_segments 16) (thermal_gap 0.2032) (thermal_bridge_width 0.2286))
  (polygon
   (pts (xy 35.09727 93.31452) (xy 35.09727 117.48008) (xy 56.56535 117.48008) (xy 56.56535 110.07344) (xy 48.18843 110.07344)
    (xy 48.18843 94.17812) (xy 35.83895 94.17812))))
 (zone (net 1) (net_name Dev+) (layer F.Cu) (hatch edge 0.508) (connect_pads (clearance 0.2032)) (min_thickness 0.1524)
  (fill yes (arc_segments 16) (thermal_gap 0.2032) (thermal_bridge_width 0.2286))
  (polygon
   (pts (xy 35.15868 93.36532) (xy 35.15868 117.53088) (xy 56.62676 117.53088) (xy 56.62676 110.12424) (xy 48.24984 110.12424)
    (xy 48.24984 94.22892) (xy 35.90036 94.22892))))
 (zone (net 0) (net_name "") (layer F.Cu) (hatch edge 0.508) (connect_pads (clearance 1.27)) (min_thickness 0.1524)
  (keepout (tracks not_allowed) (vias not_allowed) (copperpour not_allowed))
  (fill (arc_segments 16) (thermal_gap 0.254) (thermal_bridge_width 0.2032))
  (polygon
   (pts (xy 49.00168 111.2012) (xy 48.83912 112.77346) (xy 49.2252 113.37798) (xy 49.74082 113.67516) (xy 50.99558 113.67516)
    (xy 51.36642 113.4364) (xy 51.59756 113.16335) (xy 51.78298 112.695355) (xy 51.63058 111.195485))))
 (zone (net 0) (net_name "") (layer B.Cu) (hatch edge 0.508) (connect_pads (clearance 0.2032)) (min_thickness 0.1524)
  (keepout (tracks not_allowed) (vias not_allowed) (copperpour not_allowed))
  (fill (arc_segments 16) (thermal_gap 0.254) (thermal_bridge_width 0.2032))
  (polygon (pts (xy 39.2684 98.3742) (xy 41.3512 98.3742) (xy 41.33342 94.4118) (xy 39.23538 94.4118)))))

